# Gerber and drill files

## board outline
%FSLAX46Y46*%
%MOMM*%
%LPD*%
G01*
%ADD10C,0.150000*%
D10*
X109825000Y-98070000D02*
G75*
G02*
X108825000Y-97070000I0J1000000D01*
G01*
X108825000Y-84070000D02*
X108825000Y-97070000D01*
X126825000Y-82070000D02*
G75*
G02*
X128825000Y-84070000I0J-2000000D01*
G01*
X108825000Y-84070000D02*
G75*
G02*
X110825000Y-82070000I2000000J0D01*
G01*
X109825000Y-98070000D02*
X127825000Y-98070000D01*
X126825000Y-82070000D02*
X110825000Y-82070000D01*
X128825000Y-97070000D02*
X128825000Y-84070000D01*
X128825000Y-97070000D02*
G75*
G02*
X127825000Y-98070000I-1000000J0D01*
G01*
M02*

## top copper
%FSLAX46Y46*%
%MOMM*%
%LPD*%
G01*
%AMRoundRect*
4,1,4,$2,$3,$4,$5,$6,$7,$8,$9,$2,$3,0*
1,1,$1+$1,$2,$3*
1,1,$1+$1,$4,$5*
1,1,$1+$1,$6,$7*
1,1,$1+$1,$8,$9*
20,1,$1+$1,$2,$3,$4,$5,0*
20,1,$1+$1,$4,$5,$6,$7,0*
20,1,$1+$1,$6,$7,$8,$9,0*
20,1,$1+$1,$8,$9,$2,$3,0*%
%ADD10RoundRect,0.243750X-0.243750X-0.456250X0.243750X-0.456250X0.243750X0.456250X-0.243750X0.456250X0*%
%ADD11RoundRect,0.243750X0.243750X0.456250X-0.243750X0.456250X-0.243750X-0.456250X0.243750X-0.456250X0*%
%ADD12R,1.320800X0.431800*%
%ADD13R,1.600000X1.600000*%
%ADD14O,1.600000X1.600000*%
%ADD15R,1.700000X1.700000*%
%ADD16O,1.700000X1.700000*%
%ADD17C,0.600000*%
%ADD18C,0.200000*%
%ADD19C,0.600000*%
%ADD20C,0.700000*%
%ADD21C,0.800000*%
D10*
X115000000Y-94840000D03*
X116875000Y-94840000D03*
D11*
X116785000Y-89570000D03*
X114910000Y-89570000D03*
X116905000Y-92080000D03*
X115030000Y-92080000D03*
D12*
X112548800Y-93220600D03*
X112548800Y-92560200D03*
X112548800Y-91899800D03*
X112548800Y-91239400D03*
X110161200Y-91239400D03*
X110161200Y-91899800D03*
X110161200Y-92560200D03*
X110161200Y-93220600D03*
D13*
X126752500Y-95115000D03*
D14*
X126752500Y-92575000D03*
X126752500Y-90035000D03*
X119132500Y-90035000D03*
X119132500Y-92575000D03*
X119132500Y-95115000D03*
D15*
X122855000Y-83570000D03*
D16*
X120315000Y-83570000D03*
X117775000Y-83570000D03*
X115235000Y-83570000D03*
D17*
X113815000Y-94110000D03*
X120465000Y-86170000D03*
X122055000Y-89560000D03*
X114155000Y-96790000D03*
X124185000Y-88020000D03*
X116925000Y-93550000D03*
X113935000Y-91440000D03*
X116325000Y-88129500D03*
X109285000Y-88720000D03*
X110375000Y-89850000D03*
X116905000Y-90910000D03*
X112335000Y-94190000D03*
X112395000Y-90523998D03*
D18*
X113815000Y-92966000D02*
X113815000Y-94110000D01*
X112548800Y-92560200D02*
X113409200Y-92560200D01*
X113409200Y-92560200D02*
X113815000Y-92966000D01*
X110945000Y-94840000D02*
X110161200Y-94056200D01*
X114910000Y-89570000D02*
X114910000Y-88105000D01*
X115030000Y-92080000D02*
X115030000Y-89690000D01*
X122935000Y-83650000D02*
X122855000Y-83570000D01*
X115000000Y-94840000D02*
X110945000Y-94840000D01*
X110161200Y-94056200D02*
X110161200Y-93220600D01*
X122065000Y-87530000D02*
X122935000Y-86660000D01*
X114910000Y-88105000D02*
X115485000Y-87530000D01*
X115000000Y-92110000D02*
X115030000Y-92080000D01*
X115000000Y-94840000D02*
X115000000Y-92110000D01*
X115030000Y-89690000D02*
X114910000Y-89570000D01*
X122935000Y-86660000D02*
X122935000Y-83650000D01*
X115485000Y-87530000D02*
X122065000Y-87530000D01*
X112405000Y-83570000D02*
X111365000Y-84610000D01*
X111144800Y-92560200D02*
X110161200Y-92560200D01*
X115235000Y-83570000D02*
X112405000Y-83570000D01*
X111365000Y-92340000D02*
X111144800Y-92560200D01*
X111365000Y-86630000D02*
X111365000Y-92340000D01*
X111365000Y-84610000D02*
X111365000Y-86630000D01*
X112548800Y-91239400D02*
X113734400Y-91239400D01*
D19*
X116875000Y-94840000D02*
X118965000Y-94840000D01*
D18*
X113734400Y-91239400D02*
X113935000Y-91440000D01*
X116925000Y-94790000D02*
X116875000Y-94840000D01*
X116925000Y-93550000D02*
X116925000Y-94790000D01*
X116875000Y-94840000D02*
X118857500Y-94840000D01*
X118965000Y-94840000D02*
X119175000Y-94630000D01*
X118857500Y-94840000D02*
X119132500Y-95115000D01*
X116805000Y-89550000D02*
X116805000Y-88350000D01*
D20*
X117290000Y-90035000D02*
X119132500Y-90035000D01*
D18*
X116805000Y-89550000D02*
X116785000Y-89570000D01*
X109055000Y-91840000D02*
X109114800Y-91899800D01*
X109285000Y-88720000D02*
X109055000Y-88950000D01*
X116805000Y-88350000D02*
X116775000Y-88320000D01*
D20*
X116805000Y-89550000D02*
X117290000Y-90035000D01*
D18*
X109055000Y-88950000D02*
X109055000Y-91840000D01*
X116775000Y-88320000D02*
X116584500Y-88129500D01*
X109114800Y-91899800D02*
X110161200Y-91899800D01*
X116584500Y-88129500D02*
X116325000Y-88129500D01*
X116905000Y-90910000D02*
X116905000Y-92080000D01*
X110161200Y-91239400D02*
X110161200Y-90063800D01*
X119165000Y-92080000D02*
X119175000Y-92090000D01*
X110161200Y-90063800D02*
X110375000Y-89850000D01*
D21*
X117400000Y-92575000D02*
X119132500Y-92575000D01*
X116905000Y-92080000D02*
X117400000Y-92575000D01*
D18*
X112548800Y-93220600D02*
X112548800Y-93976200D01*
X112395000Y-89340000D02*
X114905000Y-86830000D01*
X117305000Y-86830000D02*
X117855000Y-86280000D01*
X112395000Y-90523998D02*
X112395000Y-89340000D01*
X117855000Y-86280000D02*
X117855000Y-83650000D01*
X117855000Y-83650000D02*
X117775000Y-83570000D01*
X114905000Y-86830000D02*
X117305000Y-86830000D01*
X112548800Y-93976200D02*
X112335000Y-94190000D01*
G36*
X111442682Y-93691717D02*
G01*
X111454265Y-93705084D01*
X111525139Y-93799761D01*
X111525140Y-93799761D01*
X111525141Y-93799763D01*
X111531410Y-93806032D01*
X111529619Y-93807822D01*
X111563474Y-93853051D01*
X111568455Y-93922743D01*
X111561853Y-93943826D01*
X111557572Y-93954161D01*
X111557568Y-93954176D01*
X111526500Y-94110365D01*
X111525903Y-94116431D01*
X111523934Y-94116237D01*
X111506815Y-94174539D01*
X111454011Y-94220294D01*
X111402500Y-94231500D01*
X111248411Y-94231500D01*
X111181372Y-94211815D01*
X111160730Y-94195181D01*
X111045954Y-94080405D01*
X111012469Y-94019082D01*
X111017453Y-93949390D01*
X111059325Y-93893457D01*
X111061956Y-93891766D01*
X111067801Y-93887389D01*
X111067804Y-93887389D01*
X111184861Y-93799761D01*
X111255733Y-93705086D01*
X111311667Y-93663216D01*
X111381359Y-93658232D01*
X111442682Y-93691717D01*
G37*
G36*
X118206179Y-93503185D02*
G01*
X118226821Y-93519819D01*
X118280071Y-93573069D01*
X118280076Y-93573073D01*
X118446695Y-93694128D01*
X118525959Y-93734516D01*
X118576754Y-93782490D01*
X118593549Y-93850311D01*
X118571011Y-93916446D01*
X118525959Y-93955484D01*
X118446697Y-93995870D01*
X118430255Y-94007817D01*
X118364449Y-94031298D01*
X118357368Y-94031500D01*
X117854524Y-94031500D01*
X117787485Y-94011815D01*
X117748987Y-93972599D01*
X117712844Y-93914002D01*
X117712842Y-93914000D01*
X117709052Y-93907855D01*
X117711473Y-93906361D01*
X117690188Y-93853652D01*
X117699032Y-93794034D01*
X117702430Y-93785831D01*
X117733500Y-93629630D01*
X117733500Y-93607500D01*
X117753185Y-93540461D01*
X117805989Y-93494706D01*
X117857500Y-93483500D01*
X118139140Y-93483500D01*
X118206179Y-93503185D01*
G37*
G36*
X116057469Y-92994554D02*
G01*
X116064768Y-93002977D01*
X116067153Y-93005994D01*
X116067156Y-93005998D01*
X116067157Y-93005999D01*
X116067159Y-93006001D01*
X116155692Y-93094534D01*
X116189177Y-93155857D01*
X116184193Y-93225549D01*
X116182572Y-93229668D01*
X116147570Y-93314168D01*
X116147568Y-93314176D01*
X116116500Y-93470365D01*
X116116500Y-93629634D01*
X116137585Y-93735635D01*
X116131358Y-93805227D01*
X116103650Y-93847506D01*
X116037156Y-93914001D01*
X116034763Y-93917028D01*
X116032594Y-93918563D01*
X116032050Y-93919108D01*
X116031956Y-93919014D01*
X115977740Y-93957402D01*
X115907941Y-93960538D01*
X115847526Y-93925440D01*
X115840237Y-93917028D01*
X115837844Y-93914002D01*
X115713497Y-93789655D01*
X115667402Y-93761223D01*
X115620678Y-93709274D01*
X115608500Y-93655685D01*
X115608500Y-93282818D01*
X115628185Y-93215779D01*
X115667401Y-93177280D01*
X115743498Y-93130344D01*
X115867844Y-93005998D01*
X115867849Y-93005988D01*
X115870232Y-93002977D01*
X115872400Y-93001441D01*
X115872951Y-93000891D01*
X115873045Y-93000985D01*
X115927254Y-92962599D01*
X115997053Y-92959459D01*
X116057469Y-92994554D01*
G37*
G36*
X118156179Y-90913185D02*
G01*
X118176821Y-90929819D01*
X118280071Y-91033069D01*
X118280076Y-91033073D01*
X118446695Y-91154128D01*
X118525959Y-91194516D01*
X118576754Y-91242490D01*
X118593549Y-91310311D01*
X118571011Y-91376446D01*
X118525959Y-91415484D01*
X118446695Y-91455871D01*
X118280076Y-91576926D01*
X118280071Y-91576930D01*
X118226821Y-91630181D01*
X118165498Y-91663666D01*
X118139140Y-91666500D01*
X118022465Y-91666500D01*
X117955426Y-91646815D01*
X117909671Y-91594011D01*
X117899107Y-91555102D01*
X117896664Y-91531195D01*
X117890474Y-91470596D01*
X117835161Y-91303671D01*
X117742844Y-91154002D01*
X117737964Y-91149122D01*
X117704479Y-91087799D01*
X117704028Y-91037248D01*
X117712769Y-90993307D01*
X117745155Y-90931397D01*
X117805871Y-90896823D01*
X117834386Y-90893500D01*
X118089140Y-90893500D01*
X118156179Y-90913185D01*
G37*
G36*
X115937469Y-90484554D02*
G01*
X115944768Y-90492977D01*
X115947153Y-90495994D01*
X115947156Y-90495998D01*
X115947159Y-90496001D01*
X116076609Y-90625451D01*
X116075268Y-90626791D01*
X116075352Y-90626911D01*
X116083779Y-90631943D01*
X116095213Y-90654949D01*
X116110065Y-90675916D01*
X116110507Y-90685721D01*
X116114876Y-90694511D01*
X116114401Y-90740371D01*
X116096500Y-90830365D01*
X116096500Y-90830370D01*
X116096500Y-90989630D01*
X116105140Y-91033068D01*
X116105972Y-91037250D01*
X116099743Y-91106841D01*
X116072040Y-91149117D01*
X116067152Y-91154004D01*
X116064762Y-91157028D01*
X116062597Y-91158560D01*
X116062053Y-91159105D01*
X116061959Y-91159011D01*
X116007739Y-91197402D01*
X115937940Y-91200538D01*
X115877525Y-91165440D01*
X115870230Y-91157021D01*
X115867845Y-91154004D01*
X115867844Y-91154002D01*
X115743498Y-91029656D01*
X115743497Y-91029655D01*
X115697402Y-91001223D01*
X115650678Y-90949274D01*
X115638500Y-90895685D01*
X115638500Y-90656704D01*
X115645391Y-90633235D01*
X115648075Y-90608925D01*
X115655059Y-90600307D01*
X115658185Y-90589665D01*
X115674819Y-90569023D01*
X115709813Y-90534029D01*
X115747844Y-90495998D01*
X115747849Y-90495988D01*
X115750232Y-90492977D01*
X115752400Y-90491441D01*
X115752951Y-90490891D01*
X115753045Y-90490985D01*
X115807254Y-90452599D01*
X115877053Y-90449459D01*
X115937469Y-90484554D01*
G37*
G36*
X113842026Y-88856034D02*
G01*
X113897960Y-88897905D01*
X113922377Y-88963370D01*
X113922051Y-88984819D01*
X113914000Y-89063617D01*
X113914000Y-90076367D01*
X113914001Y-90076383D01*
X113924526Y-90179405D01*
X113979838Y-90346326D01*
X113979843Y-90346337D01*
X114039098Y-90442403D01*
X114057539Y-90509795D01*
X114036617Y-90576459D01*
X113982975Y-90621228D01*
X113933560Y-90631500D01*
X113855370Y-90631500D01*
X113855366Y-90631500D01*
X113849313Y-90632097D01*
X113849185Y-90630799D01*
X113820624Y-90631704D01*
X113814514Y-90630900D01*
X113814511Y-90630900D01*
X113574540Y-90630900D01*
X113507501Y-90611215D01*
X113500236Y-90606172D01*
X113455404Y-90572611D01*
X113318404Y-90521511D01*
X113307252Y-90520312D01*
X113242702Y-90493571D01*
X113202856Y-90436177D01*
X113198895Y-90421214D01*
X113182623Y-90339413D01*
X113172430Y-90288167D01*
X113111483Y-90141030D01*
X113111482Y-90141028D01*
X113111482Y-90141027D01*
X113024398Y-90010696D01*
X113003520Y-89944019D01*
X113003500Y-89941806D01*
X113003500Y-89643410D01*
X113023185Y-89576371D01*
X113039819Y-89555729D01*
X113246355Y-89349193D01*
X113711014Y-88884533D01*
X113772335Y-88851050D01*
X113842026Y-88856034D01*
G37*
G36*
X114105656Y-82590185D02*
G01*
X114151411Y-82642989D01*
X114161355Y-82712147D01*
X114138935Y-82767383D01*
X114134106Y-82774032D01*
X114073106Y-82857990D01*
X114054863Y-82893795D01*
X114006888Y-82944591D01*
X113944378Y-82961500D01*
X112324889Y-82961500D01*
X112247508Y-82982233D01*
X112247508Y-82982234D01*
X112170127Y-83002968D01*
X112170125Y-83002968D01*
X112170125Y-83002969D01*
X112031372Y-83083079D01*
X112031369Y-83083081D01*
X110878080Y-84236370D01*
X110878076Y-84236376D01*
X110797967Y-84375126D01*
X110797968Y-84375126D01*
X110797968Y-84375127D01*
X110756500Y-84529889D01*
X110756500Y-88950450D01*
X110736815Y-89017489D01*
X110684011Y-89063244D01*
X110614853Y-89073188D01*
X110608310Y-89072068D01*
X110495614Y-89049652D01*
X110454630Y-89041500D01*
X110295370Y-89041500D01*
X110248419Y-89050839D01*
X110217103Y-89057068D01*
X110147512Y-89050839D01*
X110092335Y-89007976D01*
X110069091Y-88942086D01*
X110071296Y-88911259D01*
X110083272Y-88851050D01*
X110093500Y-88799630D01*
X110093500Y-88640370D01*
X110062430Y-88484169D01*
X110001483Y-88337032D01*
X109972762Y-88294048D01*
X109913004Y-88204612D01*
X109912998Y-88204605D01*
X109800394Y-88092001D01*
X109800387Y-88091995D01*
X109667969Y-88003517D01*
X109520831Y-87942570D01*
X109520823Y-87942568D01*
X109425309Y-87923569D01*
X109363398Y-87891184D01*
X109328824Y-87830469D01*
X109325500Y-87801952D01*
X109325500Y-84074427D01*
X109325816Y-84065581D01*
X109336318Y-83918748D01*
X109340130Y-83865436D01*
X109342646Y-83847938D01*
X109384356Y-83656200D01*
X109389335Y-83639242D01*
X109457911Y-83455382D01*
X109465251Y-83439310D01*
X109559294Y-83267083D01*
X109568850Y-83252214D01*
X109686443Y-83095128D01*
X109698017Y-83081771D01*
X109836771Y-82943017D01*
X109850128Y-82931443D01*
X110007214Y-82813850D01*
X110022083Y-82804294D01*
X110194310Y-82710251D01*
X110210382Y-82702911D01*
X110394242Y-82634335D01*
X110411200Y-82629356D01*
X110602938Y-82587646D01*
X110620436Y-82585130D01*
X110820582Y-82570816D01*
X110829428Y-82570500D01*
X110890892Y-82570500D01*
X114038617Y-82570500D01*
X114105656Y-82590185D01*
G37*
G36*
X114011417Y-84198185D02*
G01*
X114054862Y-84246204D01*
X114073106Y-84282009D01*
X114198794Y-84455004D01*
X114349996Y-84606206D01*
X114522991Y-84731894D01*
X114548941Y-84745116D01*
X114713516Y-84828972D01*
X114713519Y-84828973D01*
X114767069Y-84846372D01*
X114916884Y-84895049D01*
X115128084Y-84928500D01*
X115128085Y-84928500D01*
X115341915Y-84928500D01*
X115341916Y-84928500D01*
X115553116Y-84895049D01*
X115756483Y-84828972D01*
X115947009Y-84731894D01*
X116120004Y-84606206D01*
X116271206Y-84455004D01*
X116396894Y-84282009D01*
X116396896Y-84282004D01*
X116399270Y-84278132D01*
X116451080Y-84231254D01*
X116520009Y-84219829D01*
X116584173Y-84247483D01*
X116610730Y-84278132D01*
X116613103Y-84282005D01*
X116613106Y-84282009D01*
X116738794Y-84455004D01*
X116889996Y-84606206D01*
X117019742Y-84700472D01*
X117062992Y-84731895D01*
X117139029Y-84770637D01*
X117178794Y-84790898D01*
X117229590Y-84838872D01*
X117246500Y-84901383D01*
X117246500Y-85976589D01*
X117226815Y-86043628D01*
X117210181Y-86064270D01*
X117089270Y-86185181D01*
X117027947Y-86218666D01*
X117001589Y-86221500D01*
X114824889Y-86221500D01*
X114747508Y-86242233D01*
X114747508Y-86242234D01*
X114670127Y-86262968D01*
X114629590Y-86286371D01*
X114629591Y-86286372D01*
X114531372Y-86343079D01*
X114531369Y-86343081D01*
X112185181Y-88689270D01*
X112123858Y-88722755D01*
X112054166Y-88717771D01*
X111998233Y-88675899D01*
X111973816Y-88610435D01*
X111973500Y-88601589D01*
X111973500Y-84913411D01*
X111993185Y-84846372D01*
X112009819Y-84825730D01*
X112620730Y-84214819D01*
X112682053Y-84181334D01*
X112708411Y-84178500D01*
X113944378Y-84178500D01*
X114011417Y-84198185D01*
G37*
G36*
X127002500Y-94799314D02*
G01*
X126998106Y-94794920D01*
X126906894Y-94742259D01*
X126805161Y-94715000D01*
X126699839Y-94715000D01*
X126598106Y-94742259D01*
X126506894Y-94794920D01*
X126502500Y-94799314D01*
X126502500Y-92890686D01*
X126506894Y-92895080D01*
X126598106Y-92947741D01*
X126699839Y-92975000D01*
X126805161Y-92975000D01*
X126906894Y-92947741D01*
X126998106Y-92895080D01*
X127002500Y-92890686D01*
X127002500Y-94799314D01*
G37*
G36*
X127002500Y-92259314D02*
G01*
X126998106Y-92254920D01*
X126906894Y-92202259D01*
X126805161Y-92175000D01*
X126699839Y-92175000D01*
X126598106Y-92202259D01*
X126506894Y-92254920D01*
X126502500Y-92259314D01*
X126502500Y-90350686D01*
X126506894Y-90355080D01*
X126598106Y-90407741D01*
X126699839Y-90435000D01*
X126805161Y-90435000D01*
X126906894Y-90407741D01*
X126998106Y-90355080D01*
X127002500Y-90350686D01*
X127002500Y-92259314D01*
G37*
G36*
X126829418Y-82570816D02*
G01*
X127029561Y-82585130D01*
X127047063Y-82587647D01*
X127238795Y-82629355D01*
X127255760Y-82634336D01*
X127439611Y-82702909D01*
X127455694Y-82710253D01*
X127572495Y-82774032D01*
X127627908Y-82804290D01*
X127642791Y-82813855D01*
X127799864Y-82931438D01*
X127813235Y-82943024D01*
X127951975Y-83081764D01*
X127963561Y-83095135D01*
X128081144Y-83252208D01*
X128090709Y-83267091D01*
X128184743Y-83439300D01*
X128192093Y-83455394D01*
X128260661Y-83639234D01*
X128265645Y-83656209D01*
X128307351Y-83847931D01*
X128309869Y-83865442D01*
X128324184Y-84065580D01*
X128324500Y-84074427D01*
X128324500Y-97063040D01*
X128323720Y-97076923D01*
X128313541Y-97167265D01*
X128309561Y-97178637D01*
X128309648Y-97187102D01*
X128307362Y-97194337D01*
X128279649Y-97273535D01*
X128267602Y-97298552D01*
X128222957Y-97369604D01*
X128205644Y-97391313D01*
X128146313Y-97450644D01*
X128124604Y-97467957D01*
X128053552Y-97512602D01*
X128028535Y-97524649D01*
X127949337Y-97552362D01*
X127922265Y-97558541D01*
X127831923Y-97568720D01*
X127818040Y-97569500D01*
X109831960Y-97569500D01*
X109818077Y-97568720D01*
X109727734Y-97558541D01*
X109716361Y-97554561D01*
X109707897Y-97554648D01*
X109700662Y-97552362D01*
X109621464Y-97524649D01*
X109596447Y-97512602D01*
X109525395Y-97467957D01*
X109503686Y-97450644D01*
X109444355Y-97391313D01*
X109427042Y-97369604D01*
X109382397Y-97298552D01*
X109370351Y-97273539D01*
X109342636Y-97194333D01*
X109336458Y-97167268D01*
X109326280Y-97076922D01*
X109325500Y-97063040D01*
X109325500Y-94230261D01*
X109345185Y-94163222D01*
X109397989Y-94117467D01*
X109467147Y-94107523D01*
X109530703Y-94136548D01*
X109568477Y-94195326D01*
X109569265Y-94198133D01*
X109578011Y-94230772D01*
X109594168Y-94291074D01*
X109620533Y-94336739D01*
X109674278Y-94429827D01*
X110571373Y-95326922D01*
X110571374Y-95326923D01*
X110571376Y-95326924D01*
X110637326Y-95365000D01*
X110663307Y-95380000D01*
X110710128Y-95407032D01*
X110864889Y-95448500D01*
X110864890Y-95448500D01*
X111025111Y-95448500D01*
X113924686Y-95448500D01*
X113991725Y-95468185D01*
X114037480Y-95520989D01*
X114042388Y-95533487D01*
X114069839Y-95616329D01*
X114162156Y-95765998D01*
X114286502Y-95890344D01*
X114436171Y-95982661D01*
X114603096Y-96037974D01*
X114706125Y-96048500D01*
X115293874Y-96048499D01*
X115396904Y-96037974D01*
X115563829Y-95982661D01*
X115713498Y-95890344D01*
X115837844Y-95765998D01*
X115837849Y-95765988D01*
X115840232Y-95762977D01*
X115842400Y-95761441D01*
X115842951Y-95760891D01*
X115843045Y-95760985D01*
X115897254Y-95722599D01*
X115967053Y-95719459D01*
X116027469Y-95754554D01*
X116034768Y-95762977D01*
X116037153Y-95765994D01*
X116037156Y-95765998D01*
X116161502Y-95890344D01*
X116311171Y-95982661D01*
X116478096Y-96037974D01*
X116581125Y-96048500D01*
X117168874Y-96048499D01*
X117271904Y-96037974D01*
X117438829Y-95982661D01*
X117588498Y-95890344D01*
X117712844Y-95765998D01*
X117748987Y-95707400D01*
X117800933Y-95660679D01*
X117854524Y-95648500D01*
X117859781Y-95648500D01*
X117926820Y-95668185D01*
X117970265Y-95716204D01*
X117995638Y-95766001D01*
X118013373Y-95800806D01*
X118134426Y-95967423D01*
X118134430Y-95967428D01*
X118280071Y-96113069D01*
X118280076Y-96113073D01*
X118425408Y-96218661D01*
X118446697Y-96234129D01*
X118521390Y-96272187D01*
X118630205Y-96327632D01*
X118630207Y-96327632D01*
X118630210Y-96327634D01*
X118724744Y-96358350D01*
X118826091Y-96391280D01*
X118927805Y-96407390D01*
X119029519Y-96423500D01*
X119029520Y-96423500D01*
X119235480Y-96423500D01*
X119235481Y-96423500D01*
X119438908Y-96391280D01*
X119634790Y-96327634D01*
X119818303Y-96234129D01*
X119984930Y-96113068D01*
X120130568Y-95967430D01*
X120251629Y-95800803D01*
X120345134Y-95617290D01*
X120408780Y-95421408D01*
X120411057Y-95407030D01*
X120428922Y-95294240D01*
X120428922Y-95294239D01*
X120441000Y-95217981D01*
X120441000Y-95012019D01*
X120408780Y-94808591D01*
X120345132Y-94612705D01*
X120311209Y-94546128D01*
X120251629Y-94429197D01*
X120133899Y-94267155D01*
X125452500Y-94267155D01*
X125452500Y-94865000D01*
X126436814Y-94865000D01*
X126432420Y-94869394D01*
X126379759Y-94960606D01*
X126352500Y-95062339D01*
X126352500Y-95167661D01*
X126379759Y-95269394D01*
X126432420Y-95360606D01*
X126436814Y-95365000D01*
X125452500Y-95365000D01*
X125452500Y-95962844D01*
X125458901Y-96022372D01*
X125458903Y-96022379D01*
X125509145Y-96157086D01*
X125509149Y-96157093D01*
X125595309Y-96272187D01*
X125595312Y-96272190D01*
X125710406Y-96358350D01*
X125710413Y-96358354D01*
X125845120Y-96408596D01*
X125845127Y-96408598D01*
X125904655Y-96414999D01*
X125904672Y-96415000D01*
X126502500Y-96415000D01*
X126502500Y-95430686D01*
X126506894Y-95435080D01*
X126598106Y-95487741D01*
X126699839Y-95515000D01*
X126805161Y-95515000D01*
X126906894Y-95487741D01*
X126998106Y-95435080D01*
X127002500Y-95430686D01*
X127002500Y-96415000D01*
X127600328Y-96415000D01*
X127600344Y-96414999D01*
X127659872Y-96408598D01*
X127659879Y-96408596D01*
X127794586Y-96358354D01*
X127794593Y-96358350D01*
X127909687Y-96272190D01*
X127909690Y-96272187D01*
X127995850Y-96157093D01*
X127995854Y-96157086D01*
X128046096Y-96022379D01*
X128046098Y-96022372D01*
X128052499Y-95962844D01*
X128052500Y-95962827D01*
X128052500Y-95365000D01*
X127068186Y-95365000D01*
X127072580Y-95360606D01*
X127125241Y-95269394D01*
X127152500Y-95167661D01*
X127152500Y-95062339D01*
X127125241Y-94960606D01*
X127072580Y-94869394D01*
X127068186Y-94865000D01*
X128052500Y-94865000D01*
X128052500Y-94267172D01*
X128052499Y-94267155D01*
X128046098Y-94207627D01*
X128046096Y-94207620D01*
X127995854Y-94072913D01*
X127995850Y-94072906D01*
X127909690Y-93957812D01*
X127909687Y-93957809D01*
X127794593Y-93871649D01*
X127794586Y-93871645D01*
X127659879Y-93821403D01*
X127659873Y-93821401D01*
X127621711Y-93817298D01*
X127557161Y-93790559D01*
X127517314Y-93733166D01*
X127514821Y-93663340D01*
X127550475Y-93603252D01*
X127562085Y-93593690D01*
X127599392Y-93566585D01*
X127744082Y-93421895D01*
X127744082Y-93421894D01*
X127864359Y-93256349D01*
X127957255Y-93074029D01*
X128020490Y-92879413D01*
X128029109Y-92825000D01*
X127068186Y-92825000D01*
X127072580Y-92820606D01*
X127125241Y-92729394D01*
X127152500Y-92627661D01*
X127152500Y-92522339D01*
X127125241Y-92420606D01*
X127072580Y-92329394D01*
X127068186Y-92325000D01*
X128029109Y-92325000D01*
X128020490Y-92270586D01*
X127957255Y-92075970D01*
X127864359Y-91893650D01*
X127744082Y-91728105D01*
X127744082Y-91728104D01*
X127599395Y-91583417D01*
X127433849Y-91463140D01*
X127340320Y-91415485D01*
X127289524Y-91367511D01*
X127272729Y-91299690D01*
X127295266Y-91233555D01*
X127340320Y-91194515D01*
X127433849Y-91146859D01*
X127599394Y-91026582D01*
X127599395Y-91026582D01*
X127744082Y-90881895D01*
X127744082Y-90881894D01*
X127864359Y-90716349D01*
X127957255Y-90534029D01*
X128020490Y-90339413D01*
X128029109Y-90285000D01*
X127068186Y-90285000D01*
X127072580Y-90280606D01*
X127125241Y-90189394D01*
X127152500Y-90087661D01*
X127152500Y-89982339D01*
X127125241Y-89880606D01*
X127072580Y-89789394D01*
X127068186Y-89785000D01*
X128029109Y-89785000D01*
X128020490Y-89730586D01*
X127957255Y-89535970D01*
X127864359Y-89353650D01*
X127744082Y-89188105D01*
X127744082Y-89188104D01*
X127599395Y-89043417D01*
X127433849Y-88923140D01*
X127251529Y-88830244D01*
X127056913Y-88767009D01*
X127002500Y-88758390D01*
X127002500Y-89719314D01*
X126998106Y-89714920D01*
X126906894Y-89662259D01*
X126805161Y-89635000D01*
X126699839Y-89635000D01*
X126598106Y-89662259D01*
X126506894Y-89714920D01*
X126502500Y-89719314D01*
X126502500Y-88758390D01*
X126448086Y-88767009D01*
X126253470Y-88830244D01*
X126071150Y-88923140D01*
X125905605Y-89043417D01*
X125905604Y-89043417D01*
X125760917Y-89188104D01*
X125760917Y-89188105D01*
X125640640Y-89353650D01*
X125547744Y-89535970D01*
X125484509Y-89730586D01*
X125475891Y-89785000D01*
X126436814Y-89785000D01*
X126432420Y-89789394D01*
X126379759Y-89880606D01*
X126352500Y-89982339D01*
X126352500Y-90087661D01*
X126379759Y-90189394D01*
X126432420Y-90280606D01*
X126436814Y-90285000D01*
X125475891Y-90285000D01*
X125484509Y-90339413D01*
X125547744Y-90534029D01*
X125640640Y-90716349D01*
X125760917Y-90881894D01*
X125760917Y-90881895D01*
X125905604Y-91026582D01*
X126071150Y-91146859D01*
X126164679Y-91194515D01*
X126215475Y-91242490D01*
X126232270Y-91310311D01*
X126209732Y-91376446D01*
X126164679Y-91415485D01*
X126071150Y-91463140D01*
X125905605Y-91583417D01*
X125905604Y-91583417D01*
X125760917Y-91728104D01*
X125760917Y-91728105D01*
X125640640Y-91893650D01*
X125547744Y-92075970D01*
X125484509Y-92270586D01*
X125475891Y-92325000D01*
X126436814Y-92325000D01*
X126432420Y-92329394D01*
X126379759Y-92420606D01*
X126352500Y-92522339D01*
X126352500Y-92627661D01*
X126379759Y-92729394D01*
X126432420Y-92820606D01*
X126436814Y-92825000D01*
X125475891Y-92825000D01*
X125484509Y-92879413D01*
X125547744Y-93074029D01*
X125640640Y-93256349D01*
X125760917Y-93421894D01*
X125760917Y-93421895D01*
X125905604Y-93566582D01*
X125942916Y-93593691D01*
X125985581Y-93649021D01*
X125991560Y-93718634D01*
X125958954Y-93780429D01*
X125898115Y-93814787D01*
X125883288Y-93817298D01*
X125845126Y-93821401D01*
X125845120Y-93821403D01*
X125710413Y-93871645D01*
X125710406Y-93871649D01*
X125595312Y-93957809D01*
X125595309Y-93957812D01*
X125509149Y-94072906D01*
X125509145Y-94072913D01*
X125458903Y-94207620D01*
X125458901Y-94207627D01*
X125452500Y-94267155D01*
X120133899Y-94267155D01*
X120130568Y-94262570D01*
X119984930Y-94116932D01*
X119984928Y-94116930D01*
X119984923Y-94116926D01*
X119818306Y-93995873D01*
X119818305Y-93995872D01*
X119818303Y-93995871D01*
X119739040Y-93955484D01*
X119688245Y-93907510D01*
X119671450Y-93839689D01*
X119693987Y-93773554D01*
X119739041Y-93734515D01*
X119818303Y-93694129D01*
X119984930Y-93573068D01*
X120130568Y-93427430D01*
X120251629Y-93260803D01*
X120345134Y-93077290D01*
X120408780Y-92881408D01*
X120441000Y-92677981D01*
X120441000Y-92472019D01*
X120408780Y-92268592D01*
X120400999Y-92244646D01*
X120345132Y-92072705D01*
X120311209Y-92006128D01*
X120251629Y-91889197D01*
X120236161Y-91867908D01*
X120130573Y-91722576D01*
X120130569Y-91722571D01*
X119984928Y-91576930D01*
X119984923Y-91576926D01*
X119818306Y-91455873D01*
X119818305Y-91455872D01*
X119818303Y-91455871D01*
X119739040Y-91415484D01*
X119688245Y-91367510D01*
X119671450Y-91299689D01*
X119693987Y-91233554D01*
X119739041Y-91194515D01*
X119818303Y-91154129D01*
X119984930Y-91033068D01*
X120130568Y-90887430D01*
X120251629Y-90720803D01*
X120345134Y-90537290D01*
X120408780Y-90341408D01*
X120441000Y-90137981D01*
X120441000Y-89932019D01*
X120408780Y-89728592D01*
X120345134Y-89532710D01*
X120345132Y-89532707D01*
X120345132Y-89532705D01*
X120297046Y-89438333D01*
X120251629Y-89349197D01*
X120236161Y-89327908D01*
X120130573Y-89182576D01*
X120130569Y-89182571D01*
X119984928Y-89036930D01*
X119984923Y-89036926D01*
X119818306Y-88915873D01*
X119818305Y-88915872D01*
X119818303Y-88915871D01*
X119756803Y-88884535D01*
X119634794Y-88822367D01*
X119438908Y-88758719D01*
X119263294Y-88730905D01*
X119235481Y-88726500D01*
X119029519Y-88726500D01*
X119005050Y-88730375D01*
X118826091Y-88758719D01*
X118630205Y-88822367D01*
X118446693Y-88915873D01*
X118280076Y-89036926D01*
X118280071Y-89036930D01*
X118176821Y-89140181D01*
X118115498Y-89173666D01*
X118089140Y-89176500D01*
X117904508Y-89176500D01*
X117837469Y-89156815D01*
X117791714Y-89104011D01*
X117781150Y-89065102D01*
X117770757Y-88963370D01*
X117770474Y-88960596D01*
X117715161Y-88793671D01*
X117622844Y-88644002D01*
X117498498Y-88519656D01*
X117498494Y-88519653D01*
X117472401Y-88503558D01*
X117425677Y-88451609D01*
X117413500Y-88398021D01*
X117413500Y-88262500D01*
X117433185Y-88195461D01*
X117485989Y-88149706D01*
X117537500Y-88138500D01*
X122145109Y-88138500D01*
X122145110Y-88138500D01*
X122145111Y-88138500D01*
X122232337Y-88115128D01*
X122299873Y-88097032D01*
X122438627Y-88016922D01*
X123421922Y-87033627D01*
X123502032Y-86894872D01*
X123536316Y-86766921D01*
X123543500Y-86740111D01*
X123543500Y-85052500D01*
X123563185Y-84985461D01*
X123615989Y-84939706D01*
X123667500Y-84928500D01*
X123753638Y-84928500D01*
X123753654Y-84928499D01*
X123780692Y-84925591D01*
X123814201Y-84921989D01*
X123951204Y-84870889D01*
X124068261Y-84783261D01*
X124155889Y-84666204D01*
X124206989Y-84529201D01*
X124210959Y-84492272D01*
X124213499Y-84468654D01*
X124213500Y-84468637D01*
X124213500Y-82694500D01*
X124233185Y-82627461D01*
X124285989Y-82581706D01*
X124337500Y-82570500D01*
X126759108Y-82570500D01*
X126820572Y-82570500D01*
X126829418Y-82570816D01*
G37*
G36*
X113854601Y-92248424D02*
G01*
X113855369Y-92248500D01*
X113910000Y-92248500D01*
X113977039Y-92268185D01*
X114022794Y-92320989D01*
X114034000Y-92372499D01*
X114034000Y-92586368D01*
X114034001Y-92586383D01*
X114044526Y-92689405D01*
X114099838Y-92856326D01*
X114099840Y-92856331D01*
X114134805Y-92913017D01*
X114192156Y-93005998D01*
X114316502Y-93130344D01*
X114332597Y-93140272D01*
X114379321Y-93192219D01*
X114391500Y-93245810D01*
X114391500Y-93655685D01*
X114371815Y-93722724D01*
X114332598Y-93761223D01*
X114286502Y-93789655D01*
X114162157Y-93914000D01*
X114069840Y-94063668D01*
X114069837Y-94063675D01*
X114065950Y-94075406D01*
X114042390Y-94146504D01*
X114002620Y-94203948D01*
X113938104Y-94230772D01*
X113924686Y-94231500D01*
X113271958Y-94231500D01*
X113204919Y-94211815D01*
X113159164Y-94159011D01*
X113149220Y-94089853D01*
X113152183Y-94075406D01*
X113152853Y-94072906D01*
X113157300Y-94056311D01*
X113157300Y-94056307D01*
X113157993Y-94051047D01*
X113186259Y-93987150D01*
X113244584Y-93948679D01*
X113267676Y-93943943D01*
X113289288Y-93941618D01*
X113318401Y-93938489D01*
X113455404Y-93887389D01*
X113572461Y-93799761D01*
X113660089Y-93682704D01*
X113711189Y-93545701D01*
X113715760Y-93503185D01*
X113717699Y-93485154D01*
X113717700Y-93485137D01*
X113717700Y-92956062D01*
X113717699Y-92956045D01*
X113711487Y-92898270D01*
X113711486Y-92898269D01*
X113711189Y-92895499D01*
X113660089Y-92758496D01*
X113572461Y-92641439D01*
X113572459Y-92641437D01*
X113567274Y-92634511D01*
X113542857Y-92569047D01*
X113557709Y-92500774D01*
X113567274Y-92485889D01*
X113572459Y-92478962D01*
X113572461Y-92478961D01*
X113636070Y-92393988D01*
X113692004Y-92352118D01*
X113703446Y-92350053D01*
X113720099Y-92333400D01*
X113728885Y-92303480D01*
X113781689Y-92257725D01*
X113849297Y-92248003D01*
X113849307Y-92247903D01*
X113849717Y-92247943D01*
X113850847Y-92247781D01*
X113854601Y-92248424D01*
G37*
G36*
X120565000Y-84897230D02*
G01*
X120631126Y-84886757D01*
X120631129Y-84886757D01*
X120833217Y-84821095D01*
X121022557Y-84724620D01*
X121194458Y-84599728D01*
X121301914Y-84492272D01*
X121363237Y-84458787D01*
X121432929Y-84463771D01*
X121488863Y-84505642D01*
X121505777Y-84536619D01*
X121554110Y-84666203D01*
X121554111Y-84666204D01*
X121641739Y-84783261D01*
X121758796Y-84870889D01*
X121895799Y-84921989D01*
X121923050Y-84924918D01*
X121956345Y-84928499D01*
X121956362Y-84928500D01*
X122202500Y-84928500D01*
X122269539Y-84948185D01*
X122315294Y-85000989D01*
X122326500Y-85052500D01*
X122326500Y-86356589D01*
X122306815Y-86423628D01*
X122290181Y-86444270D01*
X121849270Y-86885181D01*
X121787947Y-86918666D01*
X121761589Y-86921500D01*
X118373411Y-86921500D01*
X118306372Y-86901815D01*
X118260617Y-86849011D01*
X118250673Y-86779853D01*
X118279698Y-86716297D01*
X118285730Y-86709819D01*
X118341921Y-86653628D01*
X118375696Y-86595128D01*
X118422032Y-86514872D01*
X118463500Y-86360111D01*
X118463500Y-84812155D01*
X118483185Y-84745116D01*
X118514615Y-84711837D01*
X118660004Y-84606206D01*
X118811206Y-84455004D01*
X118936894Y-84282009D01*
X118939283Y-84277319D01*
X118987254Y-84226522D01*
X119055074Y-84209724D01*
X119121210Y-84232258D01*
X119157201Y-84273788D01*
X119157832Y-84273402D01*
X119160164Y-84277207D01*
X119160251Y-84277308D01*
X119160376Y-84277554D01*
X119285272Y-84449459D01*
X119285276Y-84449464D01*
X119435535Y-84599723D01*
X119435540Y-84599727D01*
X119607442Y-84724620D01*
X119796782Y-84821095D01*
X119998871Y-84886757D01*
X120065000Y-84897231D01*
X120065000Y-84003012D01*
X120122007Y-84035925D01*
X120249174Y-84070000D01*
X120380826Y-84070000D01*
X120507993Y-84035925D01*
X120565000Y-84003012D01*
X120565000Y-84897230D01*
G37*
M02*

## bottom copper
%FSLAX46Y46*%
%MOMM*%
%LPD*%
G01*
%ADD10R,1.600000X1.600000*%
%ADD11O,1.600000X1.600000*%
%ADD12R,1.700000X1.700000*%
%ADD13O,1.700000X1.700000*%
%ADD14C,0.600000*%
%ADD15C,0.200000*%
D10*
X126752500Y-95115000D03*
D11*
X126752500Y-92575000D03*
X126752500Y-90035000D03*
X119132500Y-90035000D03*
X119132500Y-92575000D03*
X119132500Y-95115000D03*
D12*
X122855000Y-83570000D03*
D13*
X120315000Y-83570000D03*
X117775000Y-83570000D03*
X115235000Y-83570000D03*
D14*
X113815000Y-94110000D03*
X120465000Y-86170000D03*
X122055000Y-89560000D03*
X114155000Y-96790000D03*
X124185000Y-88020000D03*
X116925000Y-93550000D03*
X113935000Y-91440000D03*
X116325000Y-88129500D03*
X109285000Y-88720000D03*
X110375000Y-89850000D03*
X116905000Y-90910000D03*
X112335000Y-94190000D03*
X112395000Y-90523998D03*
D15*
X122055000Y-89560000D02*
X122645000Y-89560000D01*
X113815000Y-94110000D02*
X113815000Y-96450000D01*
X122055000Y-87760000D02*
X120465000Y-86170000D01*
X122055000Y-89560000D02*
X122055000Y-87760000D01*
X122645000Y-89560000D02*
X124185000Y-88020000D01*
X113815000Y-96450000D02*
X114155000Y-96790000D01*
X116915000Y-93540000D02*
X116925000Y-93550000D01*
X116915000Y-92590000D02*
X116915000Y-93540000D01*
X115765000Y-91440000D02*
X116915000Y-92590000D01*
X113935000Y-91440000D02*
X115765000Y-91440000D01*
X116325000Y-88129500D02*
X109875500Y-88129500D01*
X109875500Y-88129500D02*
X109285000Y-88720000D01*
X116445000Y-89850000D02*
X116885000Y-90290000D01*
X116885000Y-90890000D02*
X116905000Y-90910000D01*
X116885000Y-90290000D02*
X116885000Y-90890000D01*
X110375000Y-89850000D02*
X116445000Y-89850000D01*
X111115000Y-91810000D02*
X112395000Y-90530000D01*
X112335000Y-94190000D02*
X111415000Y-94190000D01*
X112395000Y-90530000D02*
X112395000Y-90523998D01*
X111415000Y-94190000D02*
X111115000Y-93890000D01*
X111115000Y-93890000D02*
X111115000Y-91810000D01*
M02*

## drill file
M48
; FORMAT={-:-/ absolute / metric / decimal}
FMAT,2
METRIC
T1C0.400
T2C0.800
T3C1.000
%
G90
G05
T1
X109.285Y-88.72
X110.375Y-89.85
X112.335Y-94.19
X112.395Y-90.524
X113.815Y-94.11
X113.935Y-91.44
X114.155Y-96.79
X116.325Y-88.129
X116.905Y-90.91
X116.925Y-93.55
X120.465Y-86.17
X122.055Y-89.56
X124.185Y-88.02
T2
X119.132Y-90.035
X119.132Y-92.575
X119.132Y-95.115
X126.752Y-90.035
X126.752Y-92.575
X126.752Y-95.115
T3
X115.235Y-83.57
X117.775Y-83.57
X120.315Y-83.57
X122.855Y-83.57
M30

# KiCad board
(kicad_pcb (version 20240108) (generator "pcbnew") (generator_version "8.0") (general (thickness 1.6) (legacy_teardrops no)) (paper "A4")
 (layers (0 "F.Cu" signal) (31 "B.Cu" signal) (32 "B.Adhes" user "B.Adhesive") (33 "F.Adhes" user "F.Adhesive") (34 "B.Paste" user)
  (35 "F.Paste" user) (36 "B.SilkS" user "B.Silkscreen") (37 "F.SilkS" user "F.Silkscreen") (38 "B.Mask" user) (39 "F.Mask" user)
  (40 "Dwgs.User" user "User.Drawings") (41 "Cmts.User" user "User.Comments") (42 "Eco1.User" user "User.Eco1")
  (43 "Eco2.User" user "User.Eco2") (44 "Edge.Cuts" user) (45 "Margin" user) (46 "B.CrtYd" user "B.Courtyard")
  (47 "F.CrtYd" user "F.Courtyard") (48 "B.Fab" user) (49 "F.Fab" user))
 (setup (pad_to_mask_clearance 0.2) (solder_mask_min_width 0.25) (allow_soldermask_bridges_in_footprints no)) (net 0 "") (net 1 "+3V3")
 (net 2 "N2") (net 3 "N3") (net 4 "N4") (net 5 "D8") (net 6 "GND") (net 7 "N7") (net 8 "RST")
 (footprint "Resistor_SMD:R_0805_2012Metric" (layer "F.Cu") (at 115.9375 94.84)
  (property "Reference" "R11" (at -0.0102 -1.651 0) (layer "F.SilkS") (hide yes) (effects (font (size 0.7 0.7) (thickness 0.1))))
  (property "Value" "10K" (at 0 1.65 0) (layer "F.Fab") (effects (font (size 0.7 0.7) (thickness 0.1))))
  (pad "1" smd roundrect (at -0.9375 0) (size 0.975 1.4) (layers "F.Cu" "F.Paste" "F.Mask") (roundrect_rratio 0.25) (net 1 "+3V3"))
  (pad "2" smd roundrect (at 0.9375 0) (size 0.975 1.4) (layers "F.Cu" "F.Paste" "F.Mask") (roundrect_rratio 0.25) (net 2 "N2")))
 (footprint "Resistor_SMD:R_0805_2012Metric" (layer "F.Cu") (at 115.8475 89.57 180)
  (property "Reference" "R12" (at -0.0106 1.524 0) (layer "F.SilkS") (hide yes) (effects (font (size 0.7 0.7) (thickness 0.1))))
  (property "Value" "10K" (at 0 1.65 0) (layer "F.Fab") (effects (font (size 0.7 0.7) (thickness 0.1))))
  (pad "1" smd roundrect (at -0.9375 0 180) (size 0.975 1.4) (layers "F.Cu" "F.Paste" "F.Mask") (roundrect_rratio 0.25) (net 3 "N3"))
  (pad "2" smd roundrect (at 0.9375 0 180) (size 0.975 1.4) (layers "F.Cu" "F.Paste" "F.Mask") (roundrect_rratio 0.25) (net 1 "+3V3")))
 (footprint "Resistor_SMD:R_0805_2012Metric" (layer "F.Cu") (at 115.9675 92.08 180)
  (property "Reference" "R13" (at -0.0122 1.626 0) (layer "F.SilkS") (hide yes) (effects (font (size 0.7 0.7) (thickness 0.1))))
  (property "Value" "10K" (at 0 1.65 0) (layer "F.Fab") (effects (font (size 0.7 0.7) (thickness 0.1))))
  (pad "1" smd roundrect (at -0.9375 0 180) (size 0.975 1.4) (layers "F.Cu" "F.Paste" "F.Mask") (roundrect_rratio 0.25) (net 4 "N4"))
  (pad "2" smd roundrect (at 0.9375 0 180) (size 0.975 1.4) (layers "F.Cu" "F.Paste" "F.Mask") (roundrect_rratio 0.25) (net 1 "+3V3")))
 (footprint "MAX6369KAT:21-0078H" (layer "F.Cu") (at 111.355 92.23 180)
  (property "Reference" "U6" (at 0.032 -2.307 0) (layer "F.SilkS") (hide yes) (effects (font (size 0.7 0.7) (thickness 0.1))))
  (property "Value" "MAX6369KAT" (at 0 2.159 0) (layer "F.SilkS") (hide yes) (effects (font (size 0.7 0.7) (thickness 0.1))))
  (pad "1" smd rect (at -1.1938 -0.9906 180) (size 1.3208 0.4318) (layers "F.Cu" "F.Paste" "F.Mask") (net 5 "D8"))
  (pad "2" smd rect (at -1.1938 -0.3302 180) (size 1.3208 0.4318) (layers "F.Cu" "F.Paste" "F.Mask") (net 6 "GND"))
  (pad "3" smd rect (at -1.1938 0.3302 180) (size 1.3208 0.4318) (layers "F.Cu" "F.Paste" "F.Mask") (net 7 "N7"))
  (pad "4" smd rect (at -1.1938 0.9906 180) (size 1.3208 0.4318) (layers "F.Cu" "F.Paste" "F.Mask") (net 2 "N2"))
  (pad "5" smd rect (at 1.1938 0.9906 180) (size 1.3208 0.4318) (layers "F.Cu" "F.Paste" "F.Mask") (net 4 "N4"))
  (pad "6" smd rect (at 1.1938 0.3302 180) (size 1.3208 0.4318) (layers "F.Cu" "F.Paste" "F.Mask") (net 3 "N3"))
  (pad "7" smd rect (at 1.1938 -0.3302 180) (size 1.3208 0.4318) (layers "F.Cu" "F.Paste" "F.Mask") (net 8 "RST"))
  (pad "8" smd rect (at 1.1938 -0.9906 180) (size 1.3208 0.4318) (layers "F.Cu" "F.Paste" "F.Mask") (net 1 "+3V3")))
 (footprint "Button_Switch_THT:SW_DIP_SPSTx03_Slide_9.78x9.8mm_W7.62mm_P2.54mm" (layer "F.Cu") (at 126.7525 95.115 180)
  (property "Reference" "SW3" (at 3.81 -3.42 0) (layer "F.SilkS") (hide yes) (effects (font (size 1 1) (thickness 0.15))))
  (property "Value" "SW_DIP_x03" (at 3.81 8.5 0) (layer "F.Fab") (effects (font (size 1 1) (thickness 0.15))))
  (pad "1" thru_hole rect (at 0 0 180) (size 1.6 1.6) (drill 0.8) (layers "*.Cu" "*.Mask") (remove_unused_layers no) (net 6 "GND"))
  (pad "2" thru_hole oval (at 0 2.54 180) (size 1.6 1.6) (drill 0.8) (layers "*.Cu" "*.Mask") (remove_unused_layers no) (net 6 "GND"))
  (pad "3" thru_hole oval (at 0 5.08 180) (size 1.6 1.6) (drill 0.8) (layers "*.Cu" "*.Mask") (remove_unused_layers no) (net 6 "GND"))
  (pad "4" thru_hole oval (at 7.62 5.08 180) (size 1.6 1.6) (drill 0.8) (layers "*.Cu" "*.Mask") (remove_unused_layers no) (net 3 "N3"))
  (pad "5" thru_hole oval (at 7.62 2.54 180) (size 1.6 1.6) (drill 0.8) (layers "*.Cu" "*.Mask") (remove_unused_layers no) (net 4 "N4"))
  (pad "6" thru_hole oval (at 7.62 0 180) (size 1.6 1.6) (drill 0.8) (layers "*.Cu" "*.Mask") (remove_unused_layers no) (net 2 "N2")))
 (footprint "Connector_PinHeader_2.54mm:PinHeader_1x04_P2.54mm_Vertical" (layer "F.Cu") (at 122.855 83.57 -90)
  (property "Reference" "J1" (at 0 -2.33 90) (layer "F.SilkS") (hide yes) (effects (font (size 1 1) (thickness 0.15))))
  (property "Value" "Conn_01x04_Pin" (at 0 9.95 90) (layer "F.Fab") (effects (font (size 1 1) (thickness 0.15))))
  (pad "1" thru_hole rect (at 0 0 270) (size 1.7 1.7) (drill 1) (layers "*.Cu" "*.Mask") (remove_unused_layers no) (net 1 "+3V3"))
  (pad "2" thru_hole oval (at 0 2.54 270) (size 1.7 1.7) (drill 1) (layers "*.Cu" "*.Mask") (remove_unused_layers no) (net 6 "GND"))
  (pad "3" thru_hole oval (at 0 5.08 270) (size 1.7 1.7) (drill 1) (layers "*.Cu" "*.Mask") (remove_unused_layers no) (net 5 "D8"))
  (pad "4" thru_hole oval (at 0 7.62 270) (size 1.7 1.7) (drill 1) (layers "*.Cu" "*.Mask") (remove_unused_layers no) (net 8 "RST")))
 (gr_arc (start 109.825 98.07) (mid 109.117893 97.777107) (end 108.825 97.07) (stroke (width 0.15) (type default)) (layer "Edge.Cuts"))
 (gr_line (start 108.825 84.07) (end 108.825 97.07) (stroke (width 0.15) (type default)) (layer "Edge.Cuts"))
 (gr_arc (start 126.825 82.07) (mid 128.239214 82.655786) (end 128.825 84.07) (stroke (width 0.15) (type default)) (layer "Edge.Cuts"))
 (gr_arc (start 108.825 84.07) (mid 109.410786 82.655786) (end 110.825 82.07) (stroke (width 0.15) (type default)) (layer "Edge.Cuts"))
 (gr_line (start 109.825 98.07) (end 127.825 98.07) (stroke (width 0.15) (type default)) (layer "Edge.Cuts"))
 (gr_line (start 126.825 82.07) (end 110.825 82.07) (stroke (width 0.15) (type default)) (layer "Edge.Cuts"))
 (gr_line (start 128.825 97.07) (end 128.825 84.07) (stroke (width 0.15) (type default)) (layer "Edge.Cuts"))
 (gr_arc (start 128.825 97.07) (mid 128.532107 97.777107) (end 127.825 98.07) (stroke (width 0.15) (type default)) (layer "Edge.Cuts"))
 (segment (start 113.815 92.966) (end 113.815 94.11) (width 0.2) (layer "F.Cu") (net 6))
 (segment (start 112.5488 92.5602) (end 113.4092 92.5602) (width 0.2) (layer "F.Cu") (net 6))
 (segment (start 113.4092 92.5602) (end 113.815 92.966) (width 0.2) (layer "F.Cu") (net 6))
 (via (at 113.815 94.11) (size 0.6) (drill 0.4) (layers "F.Cu" "B.Cu") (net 6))
 (via (at 120.465 86.17) (size 0.6) (drill 0.4) (layers "F.Cu" "B.Cu") (free yes) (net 6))
 (via (at 122.055 89.56) (size 0.6) (drill 0.4) (layers "F.Cu" "B.Cu") (free yes) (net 6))
 (via (at 114.155 96.79) (size 0.6) (drill 0.4) (layers "F.Cu" "B.Cu") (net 6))
 (via (at 124.185 88.02) (size 0.6) (drill 0.4) (layers "F.Cu" "B.Cu") (free yes) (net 6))
 (segment (start 122.055 89.56) (end 122.645 89.56) (width 0.2) (layer "B.Cu") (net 6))
 (segment (start 113.815 94.11) (end 113.815 96.45) (width 0.2) (layer "B.Cu") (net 6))
 (segment (start 122.055 87.76) (end 120.465 86.17) (width 0.2) (layer "B.Cu") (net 6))
 (segment (start 122.055 89.56) (end 122.055 87.76) (width 0.2) (layer "B.Cu") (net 6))
 (segment (start 122.645 89.56) (end 124.185 88.02) (width 0.2) (layer "B.Cu") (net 6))
 (segment (start 113.815 96.45) (end 114.155 96.79) (width 0.2) (layer "B.Cu") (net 6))
 (segment (start 110.945 94.84) (end 110.1612 94.0562) (width 0.2) (layer "F.Cu") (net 1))
 (segment (start 114.91 89.57) (end 114.91 88.105) (width 0.2) (layer "F.Cu") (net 1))
 (segment (start 115.03 92.08) (end 115.03 89.69) (width 0.2) (layer "F.Cu") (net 1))
 (segment (start 122.935 83.65) (end 122.855 83.57) (width 0.2) (layer "F.Cu") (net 1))
 (segment (start 115 94.84) (end 110.945 94.84) (width 0.2) (layer "F.Cu") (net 1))
 (segment (start 110.1612 94.0562) (end 110.1612 93.2206) (width 0.2) (layer "F.Cu") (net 1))
 (segment (start 122.065 87.53) (end 122.935 86.66) (width 0.2) (layer "F.Cu") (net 1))
 (segment (start 114.91 88.105) (end 115.485 87.53) (width 0.2) (layer "F.Cu") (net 1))
 (segment (start 115 92.11) (end 115.03 92.08) (width 0.2) (layer "F.Cu") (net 1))
 (segment (start 115 94.84) (end 115 92.11) (width 0.2) (layer "F.Cu") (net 1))
 (segment (start 115.03 89.69) (end 114.91 89.57) (width 0.2) (layer "F.Cu") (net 1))
 (segment (start 122.935 86.66) (end 122.935 83.65) (width 0.2) (layer "F.Cu") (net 1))
 (segment (start 115.485 87.53) (end 122.065 87.53) (width 0.2) (layer "F.Cu") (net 1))
 (segment (start 112.405 83.57) (end 111.365 84.61) (width 0.2) (layer "F.Cu") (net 8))
 (segment (start 111.1448 92.5602) (end 110.1612 92.5602) (width 0.2) (layer "F.Cu") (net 8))
 (segment (start 115.235 83.57) (end 112.405 83.57) (width 0.2) (layer "F.Cu") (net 8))
 (segment (start 111.365 92.34) (end 111.1448 92.5602) (width 0.2) (layer "F.Cu") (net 8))
 (segment (start 111.365 86.63) (end 111.365 92.34) (width 0.2) (layer "F.Cu") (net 8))
 (segment (start 111.365 84.61) (end 111.365 86.63) (width 0.2) (layer "F.Cu") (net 8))
 (segment (start 112.5488 91.2394) (end 113.7344 91.2394) (width 0.2) (layer "F.Cu") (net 2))
 (segment (start 116.875 94.84) (end 118.965 94.84) (width 0.6) (layer "F.Cu") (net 2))
 (segment (start 113.7344 91.2394) (end 113.935 91.44) (width 0.2) (layer "F.Cu") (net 2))
 (segment (start 116.925 94.79) (end 116.875 94.84) (width 0.2) (layer "F.Cu") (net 2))
 (segment (start 116.925 93.55) (end 116.925 94.79) (width 0.2) (layer "F.Cu") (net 2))
 (segment (start 116.875 94.84) (end 118.8575 94.84) (width 0.2) (layer "F.Cu") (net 2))
 (segment (start 118.965 94.84) (end 119.175 94.63) (width 0.2) (layer "F.Cu") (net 2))
 (segment (start 118.8575 94.84) (end 119.1325 95.115) (width 0.2) (layer "F.Cu") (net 2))
 (via (at 116.925 93.55) (size 0.6) (drill 0.4) (layers "F.Cu" "B.Cu") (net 2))
 (via (at 113.935 91.44) (size 0.6) (drill 0.4) (layers "F.Cu" "B.Cu") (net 2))
 (segment (start 116.915 93.54) (end 116.925 93.55) (width 0.2) (layer "B.Cu") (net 2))
 (segment (start 116.915 92.59) (end 116.915 93.54) (width 0.2) (layer "B.Cu") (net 2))
 (segment (start 115.765 91.44) (end 116.915 92.59) (width 0.2) (layer "B.Cu") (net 2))
 (segment (start 113.935 91.44) (end 115.765 91.44) (width 0.2) (layer "B.Cu") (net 2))
 (segment (start 116.805 89.55) (end 116.805 88.35) (width 0.2) (layer "F.Cu") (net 3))
 (segment (start 117.29 90.035) (end 119.1325 90.035) (width 0.7) (layer "F.Cu") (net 3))
 (segment (start 116.805 89.55) (end 116.785 89.57) (width 0.2) (layer "F.Cu") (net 3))
 (segment (start 109.055 91.84) (end 109.1148 91.8998) (width 0.2) (layer "F.Cu") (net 3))
 (segment (start 109.285 88.72) (end 109.055 88.95) (width 0.2) (layer "F.Cu") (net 3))
 (segment (start 116.805 88.35) (end 116.775 88.32) (width 0.2) (layer "F.Cu") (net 3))
 (segment (start 116.805 89.55) (end 117.29 90.035) (width 0.7) (layer "F.Cu") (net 3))
 (segment (start 109.055 88.95) (end 109.055 91.84) (width 0.2) (layer "F.Cu") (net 3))
 (segment (start 116.775 88.32) (end 116.5845 88.1295) (width 0.2) (layer "F.Cu") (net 3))
 (segment (start 109.1148 91.8998) (end 110.1612 91.8998) (width 0.2) (layer "F.Cu") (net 3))
 (segment (start 116.5845 88.1295) (end 116.325 88.1295) (width 0.2) (layer "F.Cu") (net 3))
 (via (at 116.325 88.1295) (size 0.6) (drill 0.4) (layers "F.Cu" "B.Cu") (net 3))
 (via (at 109.285 88.72) (size 0.6) (drill 0.4) (layers "F.Cu" "B.Cu") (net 3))
 (segment (start 116.325 88.1295) (end 109.8755 88.1295) (width 0.2) (layer "B.Cu") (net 3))
 (segment (start 109.8755 88.1295) (end 109.285 88.72) (width 0.2) (layer "B.Cu") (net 3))
 (segment (start 116.905 90.91) (end 116.905 92.08) (width 0.2) (layer "F.Cu") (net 4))
 (segment (start 110.1612 91.2394) (end 110.1612 90.0638) (width 0.2) (layer "F.Cu") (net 4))
 (segment (start 119.165 92.08) (end 119.175 92.09) (width 0.2) (layer "F.Cu") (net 4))
 (segment (start 110.1612 90.0638) (end 110.375 89.85) (width 0.2) (layer "F.Cu") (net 4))
 (segment (start 117.4 92.575) (end 119.1325 92.575) (width 0.8) (layer "F.Cu") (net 4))
 (segment (start 116.905 92.08) (end 117.4 92.575) (width 0.8) (layer "F.Cu") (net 4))
 (via (at 110.375 89.85) (size 0.6) (drill 0.4) (layers "F.Cu" "B.Cu") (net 4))
 (via (at 116.905 90.91) (size 0.6) (drill 0.4) (layers "F.Cu" "B.Cu") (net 4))
 (segment (start 116.445 89.85) (end 116.885 90.29) (width 0.2) (layer "B.Cu") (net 4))
 (segment (start 116.885 90.89) (end 116.905 90.91) (width 0.2) (layer "B.Cu") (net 4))
 (segment (start 116.885 90.29) (end 116.885 90.89) (width 0.2) (layer "B.Cu") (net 4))
 (segment (start 110.375 89.85) (end 116.445 89.85) (width 0.2) (layer "B.Cu") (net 4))
 (segment (start 112.5488 93.2206) (end 112.5488 93.9762) (width 0.2) (layer "F.Cu") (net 5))
 (segment (start 112.395 89.34) (end 114.905 86.83) (width 0.2) (layer "F.Cu") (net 5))
 (segment (start 117.305 86.83) (end 117.855 86.28) (width 0.2) (layer "F.Cu") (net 5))
 (segment (start 112.395 90.523998) (end 112.395 89.34) (width 0.2) (layer "F.Cu") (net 5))
 (segment (start 117.855 86.28) (end 117.855 83.65) (width 0.2) (layer "F.Cu") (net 5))
 (segment (start 117.855 83.65) (end 117.775 83.57) (width 0.2) (layer "F.Cu") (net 5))
 (segment (start 114.905 86.83) (end 117.305 86.83) (width 0.2) (layer "F.Cu") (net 5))
 (segment (start 112.5488 93.9762) (end 112.335 94.19) (width 0.2) (layer "F.Cu") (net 5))
 (via (at 112.335 94.19) (size 0.6) (drill 0.4) (layers "F.Cu" "B.Cu") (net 5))
 (via (at 112.395 90.523998) (size 0.6) (drill 0.4) (layers "F.Cu" "B.Cu") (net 5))
 (segment (start 111.115 91.81) (end 112.395 90.53) (width 0.2) (layer "B.Cu") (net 5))
 (segment (start 112.335 94.19) (end 111.415 94.19) (width 0.2) (layer "B.Cu") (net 5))
 (segment (start 112.395 90.53) (end 112.395 90.523998) (width 0.2) (layer "B.Cu") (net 5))
 (segment (start 111.415 94.19) (end 111.115 93.89) (width 0.2) (layer "B.Cu") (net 5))
 (segment (start 111.115 93.89) (end 111.115 91.81) (width 0.2) (layer "B.Cu") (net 5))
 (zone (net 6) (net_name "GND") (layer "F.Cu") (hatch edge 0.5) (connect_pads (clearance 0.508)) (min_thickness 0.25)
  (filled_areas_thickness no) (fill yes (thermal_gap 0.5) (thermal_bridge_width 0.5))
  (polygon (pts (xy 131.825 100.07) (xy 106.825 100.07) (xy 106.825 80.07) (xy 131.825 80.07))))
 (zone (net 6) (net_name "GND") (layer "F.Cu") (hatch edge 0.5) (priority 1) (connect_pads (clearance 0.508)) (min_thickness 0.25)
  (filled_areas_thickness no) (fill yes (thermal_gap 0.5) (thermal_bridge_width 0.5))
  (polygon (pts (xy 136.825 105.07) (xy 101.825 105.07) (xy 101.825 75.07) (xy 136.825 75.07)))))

